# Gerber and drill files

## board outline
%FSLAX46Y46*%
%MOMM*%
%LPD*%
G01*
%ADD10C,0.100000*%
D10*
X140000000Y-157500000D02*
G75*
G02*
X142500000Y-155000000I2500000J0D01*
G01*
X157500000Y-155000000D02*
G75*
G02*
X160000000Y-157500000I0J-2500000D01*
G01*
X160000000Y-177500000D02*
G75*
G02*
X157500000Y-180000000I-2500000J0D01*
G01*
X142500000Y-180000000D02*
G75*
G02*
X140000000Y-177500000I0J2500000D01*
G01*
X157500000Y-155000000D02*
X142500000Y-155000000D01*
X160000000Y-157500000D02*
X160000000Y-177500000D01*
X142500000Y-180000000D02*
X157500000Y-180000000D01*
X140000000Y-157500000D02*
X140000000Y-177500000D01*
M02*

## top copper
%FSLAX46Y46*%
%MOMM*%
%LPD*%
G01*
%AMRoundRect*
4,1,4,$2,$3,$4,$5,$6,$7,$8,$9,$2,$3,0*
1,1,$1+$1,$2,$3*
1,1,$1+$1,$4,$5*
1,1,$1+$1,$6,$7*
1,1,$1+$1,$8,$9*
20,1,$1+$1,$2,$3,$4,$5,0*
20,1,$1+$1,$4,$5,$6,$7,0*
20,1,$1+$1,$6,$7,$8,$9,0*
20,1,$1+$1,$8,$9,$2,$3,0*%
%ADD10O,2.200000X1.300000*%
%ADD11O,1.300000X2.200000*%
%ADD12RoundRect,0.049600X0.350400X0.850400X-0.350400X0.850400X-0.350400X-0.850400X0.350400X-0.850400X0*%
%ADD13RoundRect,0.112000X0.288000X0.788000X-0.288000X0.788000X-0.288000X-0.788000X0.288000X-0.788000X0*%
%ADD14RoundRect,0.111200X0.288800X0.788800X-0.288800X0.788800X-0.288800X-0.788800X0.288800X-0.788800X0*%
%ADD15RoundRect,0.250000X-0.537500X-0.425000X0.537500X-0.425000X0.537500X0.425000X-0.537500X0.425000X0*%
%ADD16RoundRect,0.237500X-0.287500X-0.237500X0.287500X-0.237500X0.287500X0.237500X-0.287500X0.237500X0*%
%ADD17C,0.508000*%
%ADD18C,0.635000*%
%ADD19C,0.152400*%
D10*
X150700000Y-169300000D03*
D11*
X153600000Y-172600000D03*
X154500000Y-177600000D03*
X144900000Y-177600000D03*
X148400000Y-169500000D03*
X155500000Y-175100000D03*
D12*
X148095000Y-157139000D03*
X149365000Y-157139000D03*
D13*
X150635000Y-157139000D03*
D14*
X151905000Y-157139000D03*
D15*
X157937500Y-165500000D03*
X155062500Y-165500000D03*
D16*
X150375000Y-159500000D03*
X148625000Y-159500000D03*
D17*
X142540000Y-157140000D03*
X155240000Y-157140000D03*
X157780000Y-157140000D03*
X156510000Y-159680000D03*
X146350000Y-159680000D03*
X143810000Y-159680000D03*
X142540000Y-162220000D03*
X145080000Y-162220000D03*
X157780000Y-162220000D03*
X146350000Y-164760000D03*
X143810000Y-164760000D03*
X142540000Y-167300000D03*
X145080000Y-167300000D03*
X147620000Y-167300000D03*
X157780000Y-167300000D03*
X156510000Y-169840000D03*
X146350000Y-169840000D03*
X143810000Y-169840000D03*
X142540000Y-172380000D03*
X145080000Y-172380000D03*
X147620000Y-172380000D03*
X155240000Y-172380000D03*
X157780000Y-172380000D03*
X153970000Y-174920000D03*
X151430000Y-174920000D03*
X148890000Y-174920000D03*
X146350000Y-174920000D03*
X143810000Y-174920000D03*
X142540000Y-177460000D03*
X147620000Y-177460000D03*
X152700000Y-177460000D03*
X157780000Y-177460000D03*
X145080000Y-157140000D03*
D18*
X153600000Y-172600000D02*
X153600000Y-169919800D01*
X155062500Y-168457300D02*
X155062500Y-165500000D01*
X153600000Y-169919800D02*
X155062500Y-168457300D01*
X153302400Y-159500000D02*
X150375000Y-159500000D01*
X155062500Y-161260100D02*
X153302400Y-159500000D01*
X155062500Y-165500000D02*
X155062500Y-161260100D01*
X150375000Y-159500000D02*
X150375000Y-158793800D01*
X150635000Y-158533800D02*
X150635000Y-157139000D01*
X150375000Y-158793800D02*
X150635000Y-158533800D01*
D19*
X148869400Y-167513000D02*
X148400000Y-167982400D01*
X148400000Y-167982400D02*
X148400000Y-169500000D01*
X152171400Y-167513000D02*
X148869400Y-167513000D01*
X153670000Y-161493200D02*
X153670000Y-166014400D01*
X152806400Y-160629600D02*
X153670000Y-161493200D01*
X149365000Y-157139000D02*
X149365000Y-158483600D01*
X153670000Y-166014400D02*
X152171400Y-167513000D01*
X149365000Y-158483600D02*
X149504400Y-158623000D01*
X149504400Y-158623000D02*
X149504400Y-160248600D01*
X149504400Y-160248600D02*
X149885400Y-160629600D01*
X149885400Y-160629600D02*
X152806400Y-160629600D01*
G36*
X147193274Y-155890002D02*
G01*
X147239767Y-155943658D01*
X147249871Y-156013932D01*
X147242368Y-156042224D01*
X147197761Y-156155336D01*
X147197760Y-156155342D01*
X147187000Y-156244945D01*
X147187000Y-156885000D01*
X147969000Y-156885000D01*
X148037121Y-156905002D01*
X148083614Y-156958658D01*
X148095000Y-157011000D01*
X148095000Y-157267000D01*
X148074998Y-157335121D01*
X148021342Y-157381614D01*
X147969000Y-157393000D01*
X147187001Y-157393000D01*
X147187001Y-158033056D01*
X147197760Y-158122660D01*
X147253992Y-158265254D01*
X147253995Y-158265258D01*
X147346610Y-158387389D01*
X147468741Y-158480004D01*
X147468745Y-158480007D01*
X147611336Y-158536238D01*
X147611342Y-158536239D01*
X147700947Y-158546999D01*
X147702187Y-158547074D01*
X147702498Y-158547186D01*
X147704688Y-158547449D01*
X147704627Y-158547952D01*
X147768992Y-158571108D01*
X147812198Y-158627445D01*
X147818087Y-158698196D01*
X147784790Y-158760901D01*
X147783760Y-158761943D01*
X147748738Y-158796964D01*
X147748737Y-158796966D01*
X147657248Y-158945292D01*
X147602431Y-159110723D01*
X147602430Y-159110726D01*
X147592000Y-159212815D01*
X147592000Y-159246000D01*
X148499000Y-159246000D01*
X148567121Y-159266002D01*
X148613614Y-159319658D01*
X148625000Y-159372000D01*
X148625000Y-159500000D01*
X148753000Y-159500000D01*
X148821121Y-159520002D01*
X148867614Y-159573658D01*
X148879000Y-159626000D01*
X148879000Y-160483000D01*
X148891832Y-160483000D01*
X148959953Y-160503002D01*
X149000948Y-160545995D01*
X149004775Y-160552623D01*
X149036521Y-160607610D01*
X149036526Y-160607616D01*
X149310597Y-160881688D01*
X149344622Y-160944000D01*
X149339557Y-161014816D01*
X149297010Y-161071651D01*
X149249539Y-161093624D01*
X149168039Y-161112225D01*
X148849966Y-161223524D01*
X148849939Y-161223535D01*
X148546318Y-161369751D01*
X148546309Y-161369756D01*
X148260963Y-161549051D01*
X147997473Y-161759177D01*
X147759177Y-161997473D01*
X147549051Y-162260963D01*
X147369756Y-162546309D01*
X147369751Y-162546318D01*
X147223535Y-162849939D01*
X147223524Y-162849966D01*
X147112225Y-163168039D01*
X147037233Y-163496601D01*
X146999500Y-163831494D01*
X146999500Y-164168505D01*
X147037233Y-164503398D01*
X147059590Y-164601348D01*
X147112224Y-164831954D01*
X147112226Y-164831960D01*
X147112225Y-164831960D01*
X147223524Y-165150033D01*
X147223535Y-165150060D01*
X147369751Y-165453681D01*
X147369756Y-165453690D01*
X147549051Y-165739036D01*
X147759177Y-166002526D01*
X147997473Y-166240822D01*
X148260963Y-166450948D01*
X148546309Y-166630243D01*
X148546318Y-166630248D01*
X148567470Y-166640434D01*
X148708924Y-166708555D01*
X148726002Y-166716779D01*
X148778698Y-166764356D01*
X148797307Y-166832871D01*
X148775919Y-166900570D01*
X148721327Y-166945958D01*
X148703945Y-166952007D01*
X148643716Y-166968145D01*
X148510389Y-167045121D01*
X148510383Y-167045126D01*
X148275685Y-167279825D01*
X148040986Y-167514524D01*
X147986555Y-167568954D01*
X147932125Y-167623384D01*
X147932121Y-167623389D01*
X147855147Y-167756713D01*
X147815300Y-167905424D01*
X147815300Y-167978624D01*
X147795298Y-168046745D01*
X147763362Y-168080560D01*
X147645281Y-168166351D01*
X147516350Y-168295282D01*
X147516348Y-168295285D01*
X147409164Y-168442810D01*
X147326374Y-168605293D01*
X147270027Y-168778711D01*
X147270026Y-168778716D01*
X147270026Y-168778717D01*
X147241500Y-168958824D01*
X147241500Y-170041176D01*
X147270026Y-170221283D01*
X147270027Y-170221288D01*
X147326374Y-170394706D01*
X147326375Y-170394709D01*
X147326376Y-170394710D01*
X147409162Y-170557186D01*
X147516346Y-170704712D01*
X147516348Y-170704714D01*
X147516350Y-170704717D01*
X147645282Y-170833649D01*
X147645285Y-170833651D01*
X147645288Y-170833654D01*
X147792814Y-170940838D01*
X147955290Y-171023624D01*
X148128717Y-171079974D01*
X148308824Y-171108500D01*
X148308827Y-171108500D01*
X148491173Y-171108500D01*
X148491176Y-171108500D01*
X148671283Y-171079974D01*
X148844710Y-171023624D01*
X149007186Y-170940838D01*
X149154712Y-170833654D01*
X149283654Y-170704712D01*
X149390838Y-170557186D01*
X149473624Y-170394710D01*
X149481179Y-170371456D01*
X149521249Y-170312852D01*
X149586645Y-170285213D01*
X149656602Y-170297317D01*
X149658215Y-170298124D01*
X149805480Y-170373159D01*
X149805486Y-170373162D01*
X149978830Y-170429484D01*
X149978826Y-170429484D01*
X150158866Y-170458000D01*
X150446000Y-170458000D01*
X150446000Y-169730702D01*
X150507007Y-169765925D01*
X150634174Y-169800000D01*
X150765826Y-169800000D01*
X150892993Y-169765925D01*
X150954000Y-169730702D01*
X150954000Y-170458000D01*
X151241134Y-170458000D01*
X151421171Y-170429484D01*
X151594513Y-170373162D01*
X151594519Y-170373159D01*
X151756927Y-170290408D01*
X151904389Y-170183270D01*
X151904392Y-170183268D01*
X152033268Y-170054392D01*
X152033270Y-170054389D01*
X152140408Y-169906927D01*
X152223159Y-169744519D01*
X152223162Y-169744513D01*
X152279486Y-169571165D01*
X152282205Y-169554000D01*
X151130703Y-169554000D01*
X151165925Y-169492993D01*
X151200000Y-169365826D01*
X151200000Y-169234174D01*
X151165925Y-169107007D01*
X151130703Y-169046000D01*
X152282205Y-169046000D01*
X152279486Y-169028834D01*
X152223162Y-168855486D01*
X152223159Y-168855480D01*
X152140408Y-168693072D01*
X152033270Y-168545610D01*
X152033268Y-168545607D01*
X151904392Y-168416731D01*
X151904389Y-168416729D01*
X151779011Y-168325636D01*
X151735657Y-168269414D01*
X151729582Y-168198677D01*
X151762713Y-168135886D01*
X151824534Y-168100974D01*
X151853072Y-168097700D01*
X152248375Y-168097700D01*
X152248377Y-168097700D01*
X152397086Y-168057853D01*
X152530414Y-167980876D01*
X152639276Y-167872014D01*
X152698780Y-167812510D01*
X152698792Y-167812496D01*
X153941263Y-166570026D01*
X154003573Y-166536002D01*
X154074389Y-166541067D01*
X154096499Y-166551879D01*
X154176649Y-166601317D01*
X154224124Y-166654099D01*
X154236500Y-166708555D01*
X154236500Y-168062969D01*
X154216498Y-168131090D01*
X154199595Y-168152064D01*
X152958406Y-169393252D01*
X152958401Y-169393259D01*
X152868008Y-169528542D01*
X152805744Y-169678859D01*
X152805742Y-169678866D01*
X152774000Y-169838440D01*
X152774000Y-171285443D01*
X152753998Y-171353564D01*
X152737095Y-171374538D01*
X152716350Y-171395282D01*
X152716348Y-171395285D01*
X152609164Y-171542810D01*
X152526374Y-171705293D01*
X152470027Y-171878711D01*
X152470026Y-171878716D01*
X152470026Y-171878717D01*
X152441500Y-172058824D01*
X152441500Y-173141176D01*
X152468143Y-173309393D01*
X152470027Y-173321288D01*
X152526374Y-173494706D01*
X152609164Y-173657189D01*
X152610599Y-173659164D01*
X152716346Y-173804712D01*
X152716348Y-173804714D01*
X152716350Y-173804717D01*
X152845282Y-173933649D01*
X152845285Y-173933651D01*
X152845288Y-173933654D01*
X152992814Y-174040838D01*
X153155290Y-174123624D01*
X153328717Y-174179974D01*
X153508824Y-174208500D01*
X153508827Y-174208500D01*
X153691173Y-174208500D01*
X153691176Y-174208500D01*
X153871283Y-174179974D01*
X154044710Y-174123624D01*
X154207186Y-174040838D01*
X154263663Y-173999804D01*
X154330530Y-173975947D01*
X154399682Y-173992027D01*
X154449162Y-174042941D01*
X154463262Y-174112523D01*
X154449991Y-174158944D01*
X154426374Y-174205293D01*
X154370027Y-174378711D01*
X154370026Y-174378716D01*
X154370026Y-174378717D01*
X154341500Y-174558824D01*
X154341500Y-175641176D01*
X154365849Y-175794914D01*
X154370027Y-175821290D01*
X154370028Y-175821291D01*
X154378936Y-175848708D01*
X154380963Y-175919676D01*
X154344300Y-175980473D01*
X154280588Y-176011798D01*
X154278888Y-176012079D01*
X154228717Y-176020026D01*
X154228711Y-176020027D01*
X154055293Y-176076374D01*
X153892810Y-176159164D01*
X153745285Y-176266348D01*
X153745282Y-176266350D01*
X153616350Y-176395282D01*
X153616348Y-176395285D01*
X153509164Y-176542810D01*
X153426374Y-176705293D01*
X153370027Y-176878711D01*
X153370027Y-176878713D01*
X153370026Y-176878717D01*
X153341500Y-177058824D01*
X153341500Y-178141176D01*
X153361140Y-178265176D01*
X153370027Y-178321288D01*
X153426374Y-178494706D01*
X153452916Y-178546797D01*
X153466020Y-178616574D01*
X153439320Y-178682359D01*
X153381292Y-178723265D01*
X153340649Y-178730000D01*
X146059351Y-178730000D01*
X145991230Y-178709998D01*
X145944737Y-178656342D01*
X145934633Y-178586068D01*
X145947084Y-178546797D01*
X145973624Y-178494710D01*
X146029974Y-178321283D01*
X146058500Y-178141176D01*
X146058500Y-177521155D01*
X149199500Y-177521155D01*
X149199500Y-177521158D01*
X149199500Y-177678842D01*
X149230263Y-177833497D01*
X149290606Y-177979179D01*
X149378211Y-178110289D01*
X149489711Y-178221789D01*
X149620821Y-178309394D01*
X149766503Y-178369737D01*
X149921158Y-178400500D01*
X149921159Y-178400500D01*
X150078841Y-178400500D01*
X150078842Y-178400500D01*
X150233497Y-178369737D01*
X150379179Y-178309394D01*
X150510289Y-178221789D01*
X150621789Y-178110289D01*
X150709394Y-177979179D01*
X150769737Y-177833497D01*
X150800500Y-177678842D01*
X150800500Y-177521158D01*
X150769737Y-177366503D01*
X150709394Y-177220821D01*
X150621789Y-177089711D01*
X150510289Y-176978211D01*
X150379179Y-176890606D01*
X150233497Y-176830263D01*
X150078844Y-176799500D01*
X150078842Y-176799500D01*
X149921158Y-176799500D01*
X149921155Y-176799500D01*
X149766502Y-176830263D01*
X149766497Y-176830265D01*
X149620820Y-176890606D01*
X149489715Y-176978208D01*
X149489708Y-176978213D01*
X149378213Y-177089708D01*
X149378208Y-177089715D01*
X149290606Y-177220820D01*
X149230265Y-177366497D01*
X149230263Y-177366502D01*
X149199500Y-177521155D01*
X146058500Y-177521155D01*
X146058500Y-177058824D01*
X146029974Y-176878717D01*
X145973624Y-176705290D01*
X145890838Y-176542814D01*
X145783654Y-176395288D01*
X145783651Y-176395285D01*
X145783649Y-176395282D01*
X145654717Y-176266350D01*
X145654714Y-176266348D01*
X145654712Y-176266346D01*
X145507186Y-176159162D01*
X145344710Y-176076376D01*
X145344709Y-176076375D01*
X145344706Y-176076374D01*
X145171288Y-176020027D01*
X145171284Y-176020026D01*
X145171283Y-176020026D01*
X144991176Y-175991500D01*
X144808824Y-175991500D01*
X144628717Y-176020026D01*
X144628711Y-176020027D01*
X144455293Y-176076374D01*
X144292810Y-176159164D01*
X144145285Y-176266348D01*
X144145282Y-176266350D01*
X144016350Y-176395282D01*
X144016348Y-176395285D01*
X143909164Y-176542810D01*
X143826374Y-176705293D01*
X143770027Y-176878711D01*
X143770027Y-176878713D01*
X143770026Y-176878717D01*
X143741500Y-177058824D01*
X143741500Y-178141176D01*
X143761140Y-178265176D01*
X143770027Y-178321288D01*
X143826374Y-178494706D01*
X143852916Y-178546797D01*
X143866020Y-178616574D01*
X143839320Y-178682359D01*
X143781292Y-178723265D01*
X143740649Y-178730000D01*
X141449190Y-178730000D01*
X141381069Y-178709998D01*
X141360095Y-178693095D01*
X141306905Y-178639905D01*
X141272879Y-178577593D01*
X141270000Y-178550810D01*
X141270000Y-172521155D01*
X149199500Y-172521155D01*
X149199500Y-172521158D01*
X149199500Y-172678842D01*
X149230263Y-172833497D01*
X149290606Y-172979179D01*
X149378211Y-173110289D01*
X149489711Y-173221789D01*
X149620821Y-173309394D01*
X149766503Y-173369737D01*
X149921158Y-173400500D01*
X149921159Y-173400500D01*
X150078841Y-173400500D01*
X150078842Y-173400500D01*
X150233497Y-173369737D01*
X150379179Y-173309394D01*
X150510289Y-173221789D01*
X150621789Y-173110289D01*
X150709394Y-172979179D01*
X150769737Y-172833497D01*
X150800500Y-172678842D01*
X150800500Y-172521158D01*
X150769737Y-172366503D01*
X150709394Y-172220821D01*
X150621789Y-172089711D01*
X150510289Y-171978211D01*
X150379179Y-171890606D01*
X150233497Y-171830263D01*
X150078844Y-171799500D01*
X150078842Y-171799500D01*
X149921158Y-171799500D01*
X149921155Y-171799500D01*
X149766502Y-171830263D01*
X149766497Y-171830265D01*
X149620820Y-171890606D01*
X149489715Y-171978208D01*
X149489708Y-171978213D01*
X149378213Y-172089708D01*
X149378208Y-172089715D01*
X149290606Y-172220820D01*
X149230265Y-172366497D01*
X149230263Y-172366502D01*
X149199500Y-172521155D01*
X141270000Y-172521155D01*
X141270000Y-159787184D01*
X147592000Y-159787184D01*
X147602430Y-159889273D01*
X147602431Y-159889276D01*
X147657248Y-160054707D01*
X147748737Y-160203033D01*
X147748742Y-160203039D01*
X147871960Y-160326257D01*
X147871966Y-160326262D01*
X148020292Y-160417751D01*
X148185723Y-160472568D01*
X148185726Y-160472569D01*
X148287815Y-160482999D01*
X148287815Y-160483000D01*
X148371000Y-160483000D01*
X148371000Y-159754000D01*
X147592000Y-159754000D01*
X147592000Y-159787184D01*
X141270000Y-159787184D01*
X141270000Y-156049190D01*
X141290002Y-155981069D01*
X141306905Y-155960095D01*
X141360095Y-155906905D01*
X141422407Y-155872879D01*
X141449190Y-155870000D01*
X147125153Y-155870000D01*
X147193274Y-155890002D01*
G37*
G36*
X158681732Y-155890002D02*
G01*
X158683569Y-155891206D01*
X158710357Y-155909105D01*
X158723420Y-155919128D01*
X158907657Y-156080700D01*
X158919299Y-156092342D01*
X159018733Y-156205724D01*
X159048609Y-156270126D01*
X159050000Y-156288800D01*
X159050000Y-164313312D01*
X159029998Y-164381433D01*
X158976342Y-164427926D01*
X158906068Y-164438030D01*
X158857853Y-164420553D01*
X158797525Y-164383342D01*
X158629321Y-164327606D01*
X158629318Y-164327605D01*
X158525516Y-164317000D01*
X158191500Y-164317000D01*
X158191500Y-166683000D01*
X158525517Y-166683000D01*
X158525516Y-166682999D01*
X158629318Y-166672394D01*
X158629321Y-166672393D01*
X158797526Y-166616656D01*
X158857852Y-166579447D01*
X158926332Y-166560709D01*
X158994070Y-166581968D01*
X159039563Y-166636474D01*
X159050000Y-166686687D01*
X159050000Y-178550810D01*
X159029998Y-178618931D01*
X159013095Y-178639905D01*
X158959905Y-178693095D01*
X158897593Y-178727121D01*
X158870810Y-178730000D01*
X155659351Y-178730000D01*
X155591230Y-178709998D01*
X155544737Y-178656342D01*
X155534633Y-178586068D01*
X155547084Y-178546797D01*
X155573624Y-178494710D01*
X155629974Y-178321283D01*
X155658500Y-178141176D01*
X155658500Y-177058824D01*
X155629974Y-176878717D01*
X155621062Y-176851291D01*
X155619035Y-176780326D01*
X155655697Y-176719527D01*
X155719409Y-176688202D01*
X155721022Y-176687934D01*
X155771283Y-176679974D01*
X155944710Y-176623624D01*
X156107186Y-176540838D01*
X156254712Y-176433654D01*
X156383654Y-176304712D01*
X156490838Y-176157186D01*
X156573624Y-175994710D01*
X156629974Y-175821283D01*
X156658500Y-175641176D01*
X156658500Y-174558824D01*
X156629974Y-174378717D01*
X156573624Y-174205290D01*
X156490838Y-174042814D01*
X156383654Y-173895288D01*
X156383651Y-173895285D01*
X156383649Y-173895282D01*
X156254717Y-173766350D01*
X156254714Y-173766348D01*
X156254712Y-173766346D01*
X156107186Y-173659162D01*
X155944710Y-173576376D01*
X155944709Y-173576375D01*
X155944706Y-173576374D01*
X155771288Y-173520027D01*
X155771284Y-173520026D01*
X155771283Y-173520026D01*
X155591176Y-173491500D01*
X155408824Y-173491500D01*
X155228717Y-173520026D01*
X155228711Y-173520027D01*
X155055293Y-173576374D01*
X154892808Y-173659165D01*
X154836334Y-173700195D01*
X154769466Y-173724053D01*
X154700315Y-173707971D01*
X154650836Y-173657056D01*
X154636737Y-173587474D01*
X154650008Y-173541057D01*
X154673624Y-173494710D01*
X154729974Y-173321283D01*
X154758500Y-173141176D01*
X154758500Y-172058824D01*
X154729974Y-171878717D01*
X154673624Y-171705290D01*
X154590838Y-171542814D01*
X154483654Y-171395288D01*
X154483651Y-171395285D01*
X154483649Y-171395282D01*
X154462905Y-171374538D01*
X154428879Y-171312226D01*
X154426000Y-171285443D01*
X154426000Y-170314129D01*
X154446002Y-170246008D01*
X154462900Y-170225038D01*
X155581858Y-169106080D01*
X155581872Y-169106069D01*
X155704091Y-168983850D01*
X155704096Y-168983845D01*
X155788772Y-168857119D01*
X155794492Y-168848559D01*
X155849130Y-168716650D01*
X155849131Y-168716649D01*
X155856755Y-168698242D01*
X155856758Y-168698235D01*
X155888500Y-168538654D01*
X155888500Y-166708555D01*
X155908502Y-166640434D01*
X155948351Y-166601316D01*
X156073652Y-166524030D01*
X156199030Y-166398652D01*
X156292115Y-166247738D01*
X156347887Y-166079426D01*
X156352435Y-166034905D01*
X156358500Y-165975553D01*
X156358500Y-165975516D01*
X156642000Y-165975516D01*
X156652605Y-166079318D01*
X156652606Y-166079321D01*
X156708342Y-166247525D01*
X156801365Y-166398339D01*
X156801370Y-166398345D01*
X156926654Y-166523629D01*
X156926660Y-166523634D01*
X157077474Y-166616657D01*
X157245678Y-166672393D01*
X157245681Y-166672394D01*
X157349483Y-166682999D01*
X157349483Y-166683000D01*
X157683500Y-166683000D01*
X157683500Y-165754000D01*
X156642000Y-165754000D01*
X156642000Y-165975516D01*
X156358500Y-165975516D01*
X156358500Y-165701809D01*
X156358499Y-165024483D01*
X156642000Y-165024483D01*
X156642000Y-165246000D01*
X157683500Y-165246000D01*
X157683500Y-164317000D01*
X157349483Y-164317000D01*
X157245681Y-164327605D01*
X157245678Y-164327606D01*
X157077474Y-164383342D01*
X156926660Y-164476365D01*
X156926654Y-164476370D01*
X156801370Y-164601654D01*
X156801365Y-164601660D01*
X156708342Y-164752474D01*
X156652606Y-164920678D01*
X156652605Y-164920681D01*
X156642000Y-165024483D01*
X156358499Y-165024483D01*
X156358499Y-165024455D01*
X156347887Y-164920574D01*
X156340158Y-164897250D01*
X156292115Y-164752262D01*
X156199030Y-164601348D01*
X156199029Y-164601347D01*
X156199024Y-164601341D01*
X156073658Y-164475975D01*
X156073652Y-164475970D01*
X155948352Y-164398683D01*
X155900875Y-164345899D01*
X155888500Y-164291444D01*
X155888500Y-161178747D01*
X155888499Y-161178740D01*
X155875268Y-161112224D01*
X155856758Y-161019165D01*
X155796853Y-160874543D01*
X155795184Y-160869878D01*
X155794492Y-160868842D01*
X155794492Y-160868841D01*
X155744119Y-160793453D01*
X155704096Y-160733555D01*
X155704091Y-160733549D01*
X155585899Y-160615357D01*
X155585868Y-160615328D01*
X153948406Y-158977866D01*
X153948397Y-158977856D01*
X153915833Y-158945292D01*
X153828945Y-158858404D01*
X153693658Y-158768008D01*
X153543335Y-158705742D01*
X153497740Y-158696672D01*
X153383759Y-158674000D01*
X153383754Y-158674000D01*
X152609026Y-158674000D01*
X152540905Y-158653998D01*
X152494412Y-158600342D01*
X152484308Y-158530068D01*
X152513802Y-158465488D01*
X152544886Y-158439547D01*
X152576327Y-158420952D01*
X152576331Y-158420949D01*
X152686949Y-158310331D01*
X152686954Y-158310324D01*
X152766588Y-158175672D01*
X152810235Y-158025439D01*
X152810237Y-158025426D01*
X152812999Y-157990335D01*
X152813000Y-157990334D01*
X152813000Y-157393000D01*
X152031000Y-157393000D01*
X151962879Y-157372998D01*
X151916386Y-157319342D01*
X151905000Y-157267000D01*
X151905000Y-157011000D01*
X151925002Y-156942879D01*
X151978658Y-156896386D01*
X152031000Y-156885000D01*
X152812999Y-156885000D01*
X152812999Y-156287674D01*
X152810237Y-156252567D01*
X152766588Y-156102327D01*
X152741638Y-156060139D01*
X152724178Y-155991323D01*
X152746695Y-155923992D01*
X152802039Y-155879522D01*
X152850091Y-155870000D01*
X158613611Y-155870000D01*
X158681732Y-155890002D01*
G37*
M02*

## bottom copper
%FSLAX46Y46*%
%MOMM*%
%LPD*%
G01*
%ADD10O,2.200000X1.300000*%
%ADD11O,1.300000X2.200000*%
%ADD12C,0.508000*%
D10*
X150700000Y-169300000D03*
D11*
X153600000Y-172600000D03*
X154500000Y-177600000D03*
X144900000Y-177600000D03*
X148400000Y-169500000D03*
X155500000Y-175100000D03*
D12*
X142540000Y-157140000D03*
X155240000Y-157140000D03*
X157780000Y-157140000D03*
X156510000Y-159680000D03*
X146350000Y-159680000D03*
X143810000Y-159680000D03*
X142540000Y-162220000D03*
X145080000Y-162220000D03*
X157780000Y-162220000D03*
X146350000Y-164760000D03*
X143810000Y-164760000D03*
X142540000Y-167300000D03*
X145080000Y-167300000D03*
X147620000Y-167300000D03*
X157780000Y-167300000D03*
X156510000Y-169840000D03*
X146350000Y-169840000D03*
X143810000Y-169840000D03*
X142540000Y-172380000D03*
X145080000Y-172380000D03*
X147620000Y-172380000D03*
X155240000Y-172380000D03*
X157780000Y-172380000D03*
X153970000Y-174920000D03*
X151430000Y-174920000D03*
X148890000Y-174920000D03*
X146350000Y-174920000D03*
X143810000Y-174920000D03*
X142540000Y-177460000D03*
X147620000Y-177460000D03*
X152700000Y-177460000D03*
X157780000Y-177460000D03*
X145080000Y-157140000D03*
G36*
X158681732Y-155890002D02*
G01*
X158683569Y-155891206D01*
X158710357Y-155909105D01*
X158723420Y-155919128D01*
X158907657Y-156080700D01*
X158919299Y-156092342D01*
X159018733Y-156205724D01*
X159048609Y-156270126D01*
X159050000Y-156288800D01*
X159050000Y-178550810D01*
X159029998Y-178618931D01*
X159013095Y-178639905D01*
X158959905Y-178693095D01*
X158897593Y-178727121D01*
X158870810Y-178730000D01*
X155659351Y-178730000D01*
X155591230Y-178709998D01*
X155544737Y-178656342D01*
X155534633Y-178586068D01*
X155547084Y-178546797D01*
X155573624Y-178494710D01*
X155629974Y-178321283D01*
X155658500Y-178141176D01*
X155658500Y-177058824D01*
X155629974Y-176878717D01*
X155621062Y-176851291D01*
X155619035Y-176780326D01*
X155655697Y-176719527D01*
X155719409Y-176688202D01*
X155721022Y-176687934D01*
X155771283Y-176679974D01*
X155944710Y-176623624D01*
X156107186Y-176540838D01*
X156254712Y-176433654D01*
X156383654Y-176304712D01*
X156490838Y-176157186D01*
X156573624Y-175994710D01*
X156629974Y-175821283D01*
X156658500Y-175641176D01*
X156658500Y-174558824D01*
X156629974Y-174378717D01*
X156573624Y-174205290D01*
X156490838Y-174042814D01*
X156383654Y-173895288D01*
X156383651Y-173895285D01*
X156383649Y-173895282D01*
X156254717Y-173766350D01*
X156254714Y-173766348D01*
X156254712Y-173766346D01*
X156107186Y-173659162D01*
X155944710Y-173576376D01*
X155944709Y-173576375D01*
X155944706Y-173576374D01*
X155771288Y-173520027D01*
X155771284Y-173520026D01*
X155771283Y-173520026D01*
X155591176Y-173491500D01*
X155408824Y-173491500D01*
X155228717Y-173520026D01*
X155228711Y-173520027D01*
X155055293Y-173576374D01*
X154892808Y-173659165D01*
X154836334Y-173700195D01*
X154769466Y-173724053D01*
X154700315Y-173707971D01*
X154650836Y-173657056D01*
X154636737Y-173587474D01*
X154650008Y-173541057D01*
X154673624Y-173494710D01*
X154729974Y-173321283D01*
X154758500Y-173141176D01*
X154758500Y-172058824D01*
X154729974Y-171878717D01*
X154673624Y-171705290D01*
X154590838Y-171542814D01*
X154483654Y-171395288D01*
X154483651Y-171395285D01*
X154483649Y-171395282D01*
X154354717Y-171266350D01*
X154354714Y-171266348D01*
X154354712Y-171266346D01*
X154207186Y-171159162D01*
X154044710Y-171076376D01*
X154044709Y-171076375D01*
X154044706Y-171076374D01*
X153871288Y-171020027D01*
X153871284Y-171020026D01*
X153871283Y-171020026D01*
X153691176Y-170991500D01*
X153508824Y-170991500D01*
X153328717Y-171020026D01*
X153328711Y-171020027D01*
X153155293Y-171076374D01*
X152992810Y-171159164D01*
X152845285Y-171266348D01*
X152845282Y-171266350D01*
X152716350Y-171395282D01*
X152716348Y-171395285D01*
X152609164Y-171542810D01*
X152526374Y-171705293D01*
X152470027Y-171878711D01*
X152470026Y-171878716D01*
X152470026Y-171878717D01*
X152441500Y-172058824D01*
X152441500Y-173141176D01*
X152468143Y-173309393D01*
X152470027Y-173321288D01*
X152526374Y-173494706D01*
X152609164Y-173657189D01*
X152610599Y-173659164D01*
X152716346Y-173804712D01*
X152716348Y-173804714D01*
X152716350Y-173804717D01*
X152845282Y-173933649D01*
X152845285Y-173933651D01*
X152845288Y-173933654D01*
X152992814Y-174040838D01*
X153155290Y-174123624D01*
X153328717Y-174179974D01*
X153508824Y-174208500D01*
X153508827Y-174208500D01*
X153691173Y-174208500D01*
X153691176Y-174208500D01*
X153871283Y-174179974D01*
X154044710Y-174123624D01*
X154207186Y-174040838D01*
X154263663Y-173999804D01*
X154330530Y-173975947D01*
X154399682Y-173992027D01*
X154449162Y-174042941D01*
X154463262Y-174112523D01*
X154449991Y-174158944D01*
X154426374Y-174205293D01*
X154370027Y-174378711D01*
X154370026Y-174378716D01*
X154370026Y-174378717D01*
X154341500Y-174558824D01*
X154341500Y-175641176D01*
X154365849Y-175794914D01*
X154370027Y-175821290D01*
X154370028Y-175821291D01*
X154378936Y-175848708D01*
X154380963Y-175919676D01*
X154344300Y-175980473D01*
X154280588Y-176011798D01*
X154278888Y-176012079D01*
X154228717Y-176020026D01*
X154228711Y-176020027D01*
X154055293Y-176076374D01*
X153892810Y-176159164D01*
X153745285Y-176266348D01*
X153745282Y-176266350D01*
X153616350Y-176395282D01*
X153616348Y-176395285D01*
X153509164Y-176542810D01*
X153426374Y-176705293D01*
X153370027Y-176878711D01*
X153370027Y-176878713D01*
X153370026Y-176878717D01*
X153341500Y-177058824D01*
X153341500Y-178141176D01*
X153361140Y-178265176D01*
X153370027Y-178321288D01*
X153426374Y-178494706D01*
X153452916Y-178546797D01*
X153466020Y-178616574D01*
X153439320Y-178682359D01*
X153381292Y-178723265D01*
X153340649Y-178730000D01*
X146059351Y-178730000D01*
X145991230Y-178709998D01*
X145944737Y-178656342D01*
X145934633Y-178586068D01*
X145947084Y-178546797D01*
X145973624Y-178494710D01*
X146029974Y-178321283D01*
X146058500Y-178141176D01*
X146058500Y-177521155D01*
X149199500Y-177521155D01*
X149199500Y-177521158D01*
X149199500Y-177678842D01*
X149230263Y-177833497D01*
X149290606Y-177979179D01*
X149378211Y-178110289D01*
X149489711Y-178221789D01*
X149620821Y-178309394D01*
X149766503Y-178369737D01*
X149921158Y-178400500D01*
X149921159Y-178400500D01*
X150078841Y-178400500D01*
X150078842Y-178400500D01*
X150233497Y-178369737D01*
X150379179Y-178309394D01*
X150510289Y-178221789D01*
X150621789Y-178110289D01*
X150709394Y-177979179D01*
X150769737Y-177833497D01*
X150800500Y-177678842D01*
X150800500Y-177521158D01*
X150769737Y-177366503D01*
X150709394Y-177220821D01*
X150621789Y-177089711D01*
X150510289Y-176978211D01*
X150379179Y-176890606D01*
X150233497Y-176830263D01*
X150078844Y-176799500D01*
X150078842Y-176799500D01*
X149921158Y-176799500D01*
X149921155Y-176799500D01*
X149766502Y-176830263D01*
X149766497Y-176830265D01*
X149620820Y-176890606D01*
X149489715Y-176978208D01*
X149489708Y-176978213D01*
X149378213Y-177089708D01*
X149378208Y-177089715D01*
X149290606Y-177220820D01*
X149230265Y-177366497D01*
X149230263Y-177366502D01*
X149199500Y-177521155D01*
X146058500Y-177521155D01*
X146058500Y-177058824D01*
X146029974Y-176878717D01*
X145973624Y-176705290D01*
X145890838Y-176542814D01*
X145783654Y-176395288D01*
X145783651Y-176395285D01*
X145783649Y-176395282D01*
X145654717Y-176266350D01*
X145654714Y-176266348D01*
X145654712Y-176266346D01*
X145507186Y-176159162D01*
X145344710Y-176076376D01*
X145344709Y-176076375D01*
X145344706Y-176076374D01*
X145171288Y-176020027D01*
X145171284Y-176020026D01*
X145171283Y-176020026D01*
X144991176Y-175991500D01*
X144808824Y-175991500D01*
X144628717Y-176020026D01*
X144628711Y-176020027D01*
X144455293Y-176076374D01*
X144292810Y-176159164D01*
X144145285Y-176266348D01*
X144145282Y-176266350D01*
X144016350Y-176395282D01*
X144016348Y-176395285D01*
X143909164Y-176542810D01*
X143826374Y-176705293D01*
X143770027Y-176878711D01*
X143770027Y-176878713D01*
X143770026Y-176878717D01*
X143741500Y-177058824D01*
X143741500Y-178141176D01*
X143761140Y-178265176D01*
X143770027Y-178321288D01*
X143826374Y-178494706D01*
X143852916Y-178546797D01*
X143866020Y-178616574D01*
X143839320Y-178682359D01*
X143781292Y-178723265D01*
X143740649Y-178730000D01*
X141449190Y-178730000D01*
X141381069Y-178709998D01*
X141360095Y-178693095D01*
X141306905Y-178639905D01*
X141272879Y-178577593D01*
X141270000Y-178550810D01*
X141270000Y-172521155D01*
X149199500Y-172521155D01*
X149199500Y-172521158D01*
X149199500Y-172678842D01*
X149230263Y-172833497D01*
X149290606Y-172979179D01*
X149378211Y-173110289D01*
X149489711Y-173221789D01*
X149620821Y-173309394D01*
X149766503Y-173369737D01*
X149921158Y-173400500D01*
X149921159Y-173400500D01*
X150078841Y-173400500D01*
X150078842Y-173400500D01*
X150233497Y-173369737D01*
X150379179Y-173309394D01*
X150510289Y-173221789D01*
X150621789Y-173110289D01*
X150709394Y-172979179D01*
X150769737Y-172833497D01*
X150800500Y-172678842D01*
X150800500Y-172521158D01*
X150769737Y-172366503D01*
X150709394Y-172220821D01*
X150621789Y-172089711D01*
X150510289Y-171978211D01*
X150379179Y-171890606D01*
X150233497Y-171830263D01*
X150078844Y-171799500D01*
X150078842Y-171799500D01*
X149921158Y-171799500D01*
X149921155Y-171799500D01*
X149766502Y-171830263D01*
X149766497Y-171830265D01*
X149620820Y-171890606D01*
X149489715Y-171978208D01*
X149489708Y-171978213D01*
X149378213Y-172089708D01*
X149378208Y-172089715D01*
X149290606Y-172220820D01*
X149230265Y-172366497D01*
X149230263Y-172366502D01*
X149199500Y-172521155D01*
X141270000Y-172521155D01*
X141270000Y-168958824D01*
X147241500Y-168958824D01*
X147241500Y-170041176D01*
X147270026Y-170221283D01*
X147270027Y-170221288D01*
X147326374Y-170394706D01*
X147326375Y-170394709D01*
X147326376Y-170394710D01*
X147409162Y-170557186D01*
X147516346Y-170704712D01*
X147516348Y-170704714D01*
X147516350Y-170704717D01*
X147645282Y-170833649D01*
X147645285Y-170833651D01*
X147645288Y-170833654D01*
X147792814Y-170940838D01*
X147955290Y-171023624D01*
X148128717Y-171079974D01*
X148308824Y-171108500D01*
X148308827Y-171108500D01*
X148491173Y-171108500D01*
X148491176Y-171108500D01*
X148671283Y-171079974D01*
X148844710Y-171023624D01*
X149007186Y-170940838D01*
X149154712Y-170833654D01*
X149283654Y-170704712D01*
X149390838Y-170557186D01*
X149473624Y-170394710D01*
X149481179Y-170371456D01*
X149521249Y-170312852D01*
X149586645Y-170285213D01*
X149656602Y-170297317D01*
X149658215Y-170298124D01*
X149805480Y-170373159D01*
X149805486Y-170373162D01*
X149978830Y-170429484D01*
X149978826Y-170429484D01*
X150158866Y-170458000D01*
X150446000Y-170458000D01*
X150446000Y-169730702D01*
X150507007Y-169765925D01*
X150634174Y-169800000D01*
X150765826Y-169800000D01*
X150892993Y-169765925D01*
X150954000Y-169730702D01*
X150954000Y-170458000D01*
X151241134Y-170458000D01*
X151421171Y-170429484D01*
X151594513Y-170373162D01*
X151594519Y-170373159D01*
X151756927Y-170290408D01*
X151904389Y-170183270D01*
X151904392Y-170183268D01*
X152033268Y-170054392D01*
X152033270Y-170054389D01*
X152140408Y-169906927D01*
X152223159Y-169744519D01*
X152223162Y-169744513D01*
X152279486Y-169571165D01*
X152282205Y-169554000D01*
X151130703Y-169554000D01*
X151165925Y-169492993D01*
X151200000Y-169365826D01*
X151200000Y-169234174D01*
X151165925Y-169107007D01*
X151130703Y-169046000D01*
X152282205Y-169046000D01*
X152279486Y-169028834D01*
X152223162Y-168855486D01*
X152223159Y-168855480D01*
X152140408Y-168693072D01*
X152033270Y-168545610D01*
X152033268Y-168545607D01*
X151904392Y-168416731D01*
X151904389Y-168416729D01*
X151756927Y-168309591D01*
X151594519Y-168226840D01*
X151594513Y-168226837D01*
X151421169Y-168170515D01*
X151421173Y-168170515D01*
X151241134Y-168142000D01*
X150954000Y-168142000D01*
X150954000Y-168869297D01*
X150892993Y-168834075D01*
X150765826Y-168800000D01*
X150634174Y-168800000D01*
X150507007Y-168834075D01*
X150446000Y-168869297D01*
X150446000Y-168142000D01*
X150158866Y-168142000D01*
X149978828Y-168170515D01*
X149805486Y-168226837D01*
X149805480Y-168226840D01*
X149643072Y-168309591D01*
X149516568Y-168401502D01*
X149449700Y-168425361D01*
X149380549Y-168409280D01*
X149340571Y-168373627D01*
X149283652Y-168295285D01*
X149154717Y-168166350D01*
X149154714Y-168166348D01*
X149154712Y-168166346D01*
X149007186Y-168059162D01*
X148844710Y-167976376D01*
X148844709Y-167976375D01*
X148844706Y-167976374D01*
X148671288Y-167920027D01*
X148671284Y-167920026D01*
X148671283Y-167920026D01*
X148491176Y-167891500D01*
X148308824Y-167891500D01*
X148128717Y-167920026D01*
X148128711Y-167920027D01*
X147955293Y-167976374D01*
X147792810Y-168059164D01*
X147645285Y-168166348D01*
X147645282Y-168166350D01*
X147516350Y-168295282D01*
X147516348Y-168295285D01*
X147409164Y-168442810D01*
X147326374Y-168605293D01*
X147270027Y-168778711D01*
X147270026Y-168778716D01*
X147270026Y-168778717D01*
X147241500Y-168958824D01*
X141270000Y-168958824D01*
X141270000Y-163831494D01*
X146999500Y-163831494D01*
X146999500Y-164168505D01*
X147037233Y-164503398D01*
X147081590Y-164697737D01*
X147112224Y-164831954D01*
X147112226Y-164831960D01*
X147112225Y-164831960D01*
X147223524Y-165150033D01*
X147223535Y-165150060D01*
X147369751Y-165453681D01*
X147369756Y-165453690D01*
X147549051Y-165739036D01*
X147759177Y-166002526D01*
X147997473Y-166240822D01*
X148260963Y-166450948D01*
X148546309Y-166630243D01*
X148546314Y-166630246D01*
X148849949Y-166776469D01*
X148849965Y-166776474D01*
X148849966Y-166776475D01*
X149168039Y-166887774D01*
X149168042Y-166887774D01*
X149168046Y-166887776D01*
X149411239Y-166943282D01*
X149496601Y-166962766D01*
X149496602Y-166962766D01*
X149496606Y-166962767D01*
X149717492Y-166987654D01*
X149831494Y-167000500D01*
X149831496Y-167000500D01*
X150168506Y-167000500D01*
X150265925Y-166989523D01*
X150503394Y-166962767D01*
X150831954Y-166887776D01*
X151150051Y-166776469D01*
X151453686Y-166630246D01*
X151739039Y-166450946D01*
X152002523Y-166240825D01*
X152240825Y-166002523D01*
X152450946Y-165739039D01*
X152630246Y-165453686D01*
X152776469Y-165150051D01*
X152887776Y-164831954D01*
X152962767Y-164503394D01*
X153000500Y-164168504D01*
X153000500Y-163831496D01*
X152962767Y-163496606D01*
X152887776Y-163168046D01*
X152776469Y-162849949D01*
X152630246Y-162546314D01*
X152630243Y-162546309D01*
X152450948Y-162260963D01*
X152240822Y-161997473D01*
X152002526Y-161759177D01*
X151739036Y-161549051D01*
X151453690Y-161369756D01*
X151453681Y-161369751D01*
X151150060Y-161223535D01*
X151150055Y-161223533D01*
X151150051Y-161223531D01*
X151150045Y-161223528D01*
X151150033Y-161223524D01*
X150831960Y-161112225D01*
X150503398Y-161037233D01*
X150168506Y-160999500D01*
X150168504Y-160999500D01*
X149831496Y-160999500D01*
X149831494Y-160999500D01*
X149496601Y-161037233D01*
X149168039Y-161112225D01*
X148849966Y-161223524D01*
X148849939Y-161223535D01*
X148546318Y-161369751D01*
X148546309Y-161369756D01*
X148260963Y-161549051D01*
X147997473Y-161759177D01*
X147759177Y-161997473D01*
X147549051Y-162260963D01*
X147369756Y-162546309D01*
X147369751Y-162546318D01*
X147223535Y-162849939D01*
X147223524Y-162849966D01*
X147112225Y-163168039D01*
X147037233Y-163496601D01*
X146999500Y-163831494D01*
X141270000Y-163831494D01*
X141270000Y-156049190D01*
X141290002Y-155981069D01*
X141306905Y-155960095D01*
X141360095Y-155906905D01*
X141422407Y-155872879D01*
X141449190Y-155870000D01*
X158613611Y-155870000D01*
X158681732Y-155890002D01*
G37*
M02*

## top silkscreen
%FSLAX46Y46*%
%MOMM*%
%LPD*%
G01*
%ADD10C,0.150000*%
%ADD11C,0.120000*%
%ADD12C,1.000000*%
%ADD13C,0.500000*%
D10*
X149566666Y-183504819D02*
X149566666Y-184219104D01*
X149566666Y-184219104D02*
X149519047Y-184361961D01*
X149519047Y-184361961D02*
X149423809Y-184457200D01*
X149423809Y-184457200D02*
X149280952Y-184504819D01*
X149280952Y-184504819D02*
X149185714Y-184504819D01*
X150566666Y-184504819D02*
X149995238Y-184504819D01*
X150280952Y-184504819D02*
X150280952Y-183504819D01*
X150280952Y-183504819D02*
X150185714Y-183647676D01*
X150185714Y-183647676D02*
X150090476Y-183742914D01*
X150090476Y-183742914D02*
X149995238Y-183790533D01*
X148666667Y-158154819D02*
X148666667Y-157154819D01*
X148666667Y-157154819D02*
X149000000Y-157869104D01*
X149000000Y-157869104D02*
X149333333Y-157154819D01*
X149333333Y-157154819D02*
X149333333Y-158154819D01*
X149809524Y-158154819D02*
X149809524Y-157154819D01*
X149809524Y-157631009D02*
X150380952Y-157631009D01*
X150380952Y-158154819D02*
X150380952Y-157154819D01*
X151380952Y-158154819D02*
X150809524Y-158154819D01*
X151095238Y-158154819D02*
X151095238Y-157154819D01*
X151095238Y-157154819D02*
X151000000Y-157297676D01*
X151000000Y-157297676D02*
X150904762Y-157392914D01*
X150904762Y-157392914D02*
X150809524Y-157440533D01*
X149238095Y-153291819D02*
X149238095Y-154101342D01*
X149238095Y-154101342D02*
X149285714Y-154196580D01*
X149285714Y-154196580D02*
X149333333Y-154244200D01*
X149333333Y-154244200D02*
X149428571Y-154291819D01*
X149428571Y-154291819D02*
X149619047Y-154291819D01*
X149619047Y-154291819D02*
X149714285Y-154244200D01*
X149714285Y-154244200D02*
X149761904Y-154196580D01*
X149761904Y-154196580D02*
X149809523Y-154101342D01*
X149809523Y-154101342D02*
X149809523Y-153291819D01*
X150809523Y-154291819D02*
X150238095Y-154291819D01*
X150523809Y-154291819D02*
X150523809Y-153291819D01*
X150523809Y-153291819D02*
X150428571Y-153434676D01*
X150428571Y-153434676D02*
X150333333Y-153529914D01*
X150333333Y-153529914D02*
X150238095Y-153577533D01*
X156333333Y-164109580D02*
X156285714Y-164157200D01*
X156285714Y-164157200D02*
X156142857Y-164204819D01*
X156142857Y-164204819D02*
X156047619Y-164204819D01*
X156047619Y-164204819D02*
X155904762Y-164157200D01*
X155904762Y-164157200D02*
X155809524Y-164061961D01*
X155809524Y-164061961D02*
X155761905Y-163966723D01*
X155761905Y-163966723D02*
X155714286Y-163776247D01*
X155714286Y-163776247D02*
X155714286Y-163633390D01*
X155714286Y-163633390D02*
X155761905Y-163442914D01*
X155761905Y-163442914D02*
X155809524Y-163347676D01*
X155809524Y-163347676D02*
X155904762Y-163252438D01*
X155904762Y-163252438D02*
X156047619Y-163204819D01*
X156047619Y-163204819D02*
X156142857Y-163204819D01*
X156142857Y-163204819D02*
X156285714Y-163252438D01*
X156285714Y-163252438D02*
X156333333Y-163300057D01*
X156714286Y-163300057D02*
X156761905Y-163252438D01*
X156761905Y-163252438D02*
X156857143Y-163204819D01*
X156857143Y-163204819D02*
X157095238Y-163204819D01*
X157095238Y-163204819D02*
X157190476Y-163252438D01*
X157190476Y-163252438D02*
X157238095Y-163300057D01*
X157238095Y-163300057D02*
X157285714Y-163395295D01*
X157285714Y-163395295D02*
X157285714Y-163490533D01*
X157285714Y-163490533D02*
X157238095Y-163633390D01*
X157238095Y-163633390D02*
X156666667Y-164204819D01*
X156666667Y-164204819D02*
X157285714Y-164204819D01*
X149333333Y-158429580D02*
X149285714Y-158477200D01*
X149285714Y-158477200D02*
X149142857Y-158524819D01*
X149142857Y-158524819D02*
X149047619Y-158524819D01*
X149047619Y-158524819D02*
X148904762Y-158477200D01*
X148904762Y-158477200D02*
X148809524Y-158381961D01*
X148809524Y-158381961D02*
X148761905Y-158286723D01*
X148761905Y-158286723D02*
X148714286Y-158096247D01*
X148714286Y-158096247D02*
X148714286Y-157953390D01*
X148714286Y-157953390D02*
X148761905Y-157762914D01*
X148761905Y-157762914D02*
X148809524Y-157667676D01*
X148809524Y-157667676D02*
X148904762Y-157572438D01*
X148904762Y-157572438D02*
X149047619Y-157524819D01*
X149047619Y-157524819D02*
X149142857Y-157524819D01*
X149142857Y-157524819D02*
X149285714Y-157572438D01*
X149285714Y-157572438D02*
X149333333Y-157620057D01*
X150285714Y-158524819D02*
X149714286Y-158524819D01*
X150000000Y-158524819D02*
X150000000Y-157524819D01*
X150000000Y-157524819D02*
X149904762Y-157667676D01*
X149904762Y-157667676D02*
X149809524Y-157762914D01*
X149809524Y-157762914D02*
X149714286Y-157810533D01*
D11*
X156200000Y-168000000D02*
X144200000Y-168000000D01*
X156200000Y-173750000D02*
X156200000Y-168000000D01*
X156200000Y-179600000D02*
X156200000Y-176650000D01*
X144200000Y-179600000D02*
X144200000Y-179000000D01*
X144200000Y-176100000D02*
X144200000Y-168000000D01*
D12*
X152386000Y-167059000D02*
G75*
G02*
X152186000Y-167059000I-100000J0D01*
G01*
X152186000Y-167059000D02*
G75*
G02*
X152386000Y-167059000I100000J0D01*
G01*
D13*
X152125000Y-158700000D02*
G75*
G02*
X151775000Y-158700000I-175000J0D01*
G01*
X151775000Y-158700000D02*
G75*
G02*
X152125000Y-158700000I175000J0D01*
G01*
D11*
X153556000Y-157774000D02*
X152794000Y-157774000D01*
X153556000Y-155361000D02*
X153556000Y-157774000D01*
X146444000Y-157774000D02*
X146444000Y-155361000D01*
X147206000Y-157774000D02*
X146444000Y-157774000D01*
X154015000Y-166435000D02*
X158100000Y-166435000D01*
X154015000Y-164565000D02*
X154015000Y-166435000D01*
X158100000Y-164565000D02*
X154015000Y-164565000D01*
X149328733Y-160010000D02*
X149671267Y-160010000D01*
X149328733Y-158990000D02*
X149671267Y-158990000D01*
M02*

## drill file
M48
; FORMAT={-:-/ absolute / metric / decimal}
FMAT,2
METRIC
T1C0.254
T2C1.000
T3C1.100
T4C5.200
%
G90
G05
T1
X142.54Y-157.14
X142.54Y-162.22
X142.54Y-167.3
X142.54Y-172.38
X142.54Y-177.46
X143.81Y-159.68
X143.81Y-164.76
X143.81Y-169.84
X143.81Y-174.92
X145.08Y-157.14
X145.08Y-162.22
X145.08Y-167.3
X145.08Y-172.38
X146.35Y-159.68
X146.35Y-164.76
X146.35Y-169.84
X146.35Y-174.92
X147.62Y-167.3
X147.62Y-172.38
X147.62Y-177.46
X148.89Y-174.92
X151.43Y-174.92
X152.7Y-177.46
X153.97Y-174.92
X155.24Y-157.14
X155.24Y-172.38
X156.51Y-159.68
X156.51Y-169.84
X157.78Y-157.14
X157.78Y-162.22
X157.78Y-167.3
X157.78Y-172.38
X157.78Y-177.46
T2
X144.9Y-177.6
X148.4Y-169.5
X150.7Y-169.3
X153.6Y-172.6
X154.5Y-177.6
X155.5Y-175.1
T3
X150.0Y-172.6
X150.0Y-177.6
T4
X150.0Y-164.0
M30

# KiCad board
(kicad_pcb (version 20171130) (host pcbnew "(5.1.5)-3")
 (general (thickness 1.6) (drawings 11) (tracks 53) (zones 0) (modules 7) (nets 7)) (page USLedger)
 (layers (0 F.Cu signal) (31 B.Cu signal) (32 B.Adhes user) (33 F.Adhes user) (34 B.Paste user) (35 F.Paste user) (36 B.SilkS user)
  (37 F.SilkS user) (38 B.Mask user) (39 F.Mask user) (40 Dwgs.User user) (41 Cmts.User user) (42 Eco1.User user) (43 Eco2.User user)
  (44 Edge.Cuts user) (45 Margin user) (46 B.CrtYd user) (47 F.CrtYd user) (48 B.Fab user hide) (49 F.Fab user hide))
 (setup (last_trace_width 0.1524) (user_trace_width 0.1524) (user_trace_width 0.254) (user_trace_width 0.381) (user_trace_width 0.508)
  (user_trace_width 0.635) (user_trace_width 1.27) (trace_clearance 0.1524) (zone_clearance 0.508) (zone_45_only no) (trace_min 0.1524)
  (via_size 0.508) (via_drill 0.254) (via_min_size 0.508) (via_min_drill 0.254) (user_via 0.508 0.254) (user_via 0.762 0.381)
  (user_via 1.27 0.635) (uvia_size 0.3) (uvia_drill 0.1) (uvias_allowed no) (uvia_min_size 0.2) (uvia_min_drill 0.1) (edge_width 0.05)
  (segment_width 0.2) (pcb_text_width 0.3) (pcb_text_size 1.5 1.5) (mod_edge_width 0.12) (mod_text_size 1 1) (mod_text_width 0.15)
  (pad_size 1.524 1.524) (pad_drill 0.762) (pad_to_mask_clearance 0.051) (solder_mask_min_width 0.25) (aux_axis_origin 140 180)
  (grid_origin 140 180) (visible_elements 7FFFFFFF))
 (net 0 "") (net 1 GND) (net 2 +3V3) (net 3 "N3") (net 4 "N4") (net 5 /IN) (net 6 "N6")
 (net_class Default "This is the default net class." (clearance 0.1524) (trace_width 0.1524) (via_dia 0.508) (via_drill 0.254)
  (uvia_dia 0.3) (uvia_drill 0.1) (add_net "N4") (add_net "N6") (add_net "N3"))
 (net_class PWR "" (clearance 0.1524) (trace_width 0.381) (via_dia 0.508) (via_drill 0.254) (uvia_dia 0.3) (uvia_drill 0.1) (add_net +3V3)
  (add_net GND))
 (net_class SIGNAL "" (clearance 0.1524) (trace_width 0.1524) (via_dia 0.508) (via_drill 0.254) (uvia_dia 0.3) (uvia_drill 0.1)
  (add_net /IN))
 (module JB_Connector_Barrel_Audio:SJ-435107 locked (layer F.Cu) (at 150 177.6 180)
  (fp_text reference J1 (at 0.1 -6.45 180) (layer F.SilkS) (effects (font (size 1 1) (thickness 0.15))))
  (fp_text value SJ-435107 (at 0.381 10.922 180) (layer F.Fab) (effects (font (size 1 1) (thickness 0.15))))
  (fp_line (start -6.2 9.6) (end 5.8 9.6) (layer F.SilkS) (width 0.12))
  (fp_line (start -6.2 3.85) (end -6.2 9.6) (layer F.SilkS) (width 0.12))
  (fp_line (start -6.2 -2) (end -6.2 0.95) (layer F.SilkS) (width 0.12))
  (fp_line (start 5.8 -2) (end 5.8 -1.4) (layer F.SilkS) (width 0.12))
  (fp_line (start 5.8 1.5) (end 5.8 9.6) (layer F.SilkS) (width 0.12))
  (fp_circle (center -2.286 10.541) (end -2.186 10.541) (layer F.SilkS) (width 1))
  (pad S thru_hole oval (at -0.7 8.3 180) (size 2.2 1.3) (drill 1) (layers *.Cu *.Mask) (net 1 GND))
  (pad T thru_hole oval (at -3.6 5 270) (size 2.2 1.3) (drill 1) (layers *.Cu *.Mask) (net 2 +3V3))
  (pad R2 thru_hole oval (at -4.5 0 270) (size 2.2 1.3) (drill 1) (layers *.Cu *.Mask) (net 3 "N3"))
  (pad G1 thru_hole oval (at 5.1 0 270) (size 2.2 1.3) (drill 1) (layers *.Cu *.Mask) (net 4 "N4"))
  (pad R1 thru_hole oval (at 1.6 8.1 270) (size 2.2 1.3) (drill 1) (layers *.Cu *.Mask) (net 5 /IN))
  (pad "" np_thru_hole circle (at 0 0 180) (size 1.1 1.1) (drill 1.1) (layers *.Cu *.Mask))
  (pad "" np_thru_hole circle (at 0 5 180) (size 1.1 1.1) (drill 1.1) (layers *.Cu *.Mask))
  (pad G2 thru_hole oval (at -5.5 2.5 270) (size 2.2 1.3) (drill 1) (layers *.Cu *.Mask) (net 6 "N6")))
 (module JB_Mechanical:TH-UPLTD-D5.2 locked (layer F.Cu) (at 150 164)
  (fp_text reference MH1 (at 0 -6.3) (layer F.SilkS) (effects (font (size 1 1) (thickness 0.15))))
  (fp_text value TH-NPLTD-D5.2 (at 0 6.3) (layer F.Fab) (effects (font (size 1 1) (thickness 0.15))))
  (pad "" np_thru_hole circle (at 0 0) (size 5.2 5.2) (drill 5.2) (layers *.Cu *.Mask) (clearance 0.4)))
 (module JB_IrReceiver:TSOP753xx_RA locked (layer F.Cu) (at 150 156.25 180)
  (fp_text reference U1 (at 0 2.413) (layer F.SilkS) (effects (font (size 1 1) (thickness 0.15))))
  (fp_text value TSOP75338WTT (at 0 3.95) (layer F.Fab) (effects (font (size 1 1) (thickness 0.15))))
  (fp_circle (center -1.95 -2.45) (end -1.775 -2.45) (layer F.SilkS) (width 0.5))
  (fp_line (start -3.556 -1.524) (end -2.794 -1.524) (layer F.SilkS) (width 0.12))
  (fp_line (start -3.556 0.889) (end -3.556 -1.524) (layer F.SilkS) (width 0.12))
  (fp_line (start 3.556 -1.524) (end 3.556 0.889) (layer F.SilkS) (width 0.12))
  (fp_line (start 2.794 -1.524) (end 3.556 -1.524) (layer F.SilkS) (width 0.12))
  (pad 4 smd roundrect (at 1.905 -0.889 180) (size 0.8 1.8) (layers F.Cu F.Paste F.Mask) (roundrect_rratio 0.062) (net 1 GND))
  (pad 3 smd roundrect (at 0.635 -0.889 180) (size 0.8 1.8) (layers F.Cu F.Paste F.Mask) (roundrect_rratio 0.062) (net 5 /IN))
  (pad 2 smd roundrect (at -0.635 -0.889 180) (size 0.8 1.8) (layers F.Cu F.Paste F.Mask) (roundrect_rratio 0.14) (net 2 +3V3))
  (pad 1 smd roundrect (at -1.905 -0.889 180) (size 0.8 1.8) (layers F.Cu F.Paste F.Mask) (roundrect_rratio 0.139) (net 1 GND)))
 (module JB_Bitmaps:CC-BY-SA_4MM (layer B.Cu) (at 143.81 169.205 180)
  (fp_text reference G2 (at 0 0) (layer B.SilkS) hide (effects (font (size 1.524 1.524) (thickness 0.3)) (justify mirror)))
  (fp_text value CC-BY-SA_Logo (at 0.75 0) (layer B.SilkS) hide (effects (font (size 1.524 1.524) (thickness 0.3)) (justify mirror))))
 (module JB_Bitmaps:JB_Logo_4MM (layer B.Cu) (at 143.937 165.268 180)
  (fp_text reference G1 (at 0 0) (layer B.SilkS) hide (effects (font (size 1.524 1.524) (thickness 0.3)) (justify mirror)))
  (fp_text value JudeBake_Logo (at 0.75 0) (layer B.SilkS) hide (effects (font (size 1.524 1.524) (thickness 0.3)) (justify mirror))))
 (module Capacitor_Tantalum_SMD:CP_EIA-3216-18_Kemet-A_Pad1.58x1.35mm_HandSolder (layer F.Cu) (at 156.5 165.5)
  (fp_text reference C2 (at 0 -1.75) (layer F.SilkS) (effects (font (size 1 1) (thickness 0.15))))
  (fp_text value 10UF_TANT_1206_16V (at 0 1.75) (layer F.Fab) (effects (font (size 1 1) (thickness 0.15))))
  (fp_line (start -2.485 0.935) (end 1.6 0.935) (layer F.SilkS) (width 0.12))
  (fp_line (start -2.485 -0.935) (end -2.485 0.935) (layer F.SilkS) (width 0.12))
  (fp_line (start 1.6 -0.935) (end -2.485 -0.935) (layer F.SilkS) (width 0.12))
  (pad 2 smd roundrect (at 1.4375 0) (size 1.575 1.35) (layers F.Cu F.Paste F.Mask) (roundrect_rratio 0.185185) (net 1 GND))
  (pad 1 smd roundrect (at -1.4375 0) (size 1.575 1.35) (layers F.Cu F.Paste F.Mask) (roundrect_rratio 0.185185) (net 2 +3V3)))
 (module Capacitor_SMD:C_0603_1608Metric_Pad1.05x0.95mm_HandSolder (layer F.Cu) (at 149.5 159.5)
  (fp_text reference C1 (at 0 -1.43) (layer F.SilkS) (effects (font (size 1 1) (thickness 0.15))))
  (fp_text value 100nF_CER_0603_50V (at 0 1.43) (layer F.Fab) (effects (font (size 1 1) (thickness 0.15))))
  (fp_line (start -0.171267 0.51) (end 0.171267 0.51) (layer F.SilkS) (width 0.12))
  (fp_line (start -0.171267 -0.51) (end 0.171267 -0.51) (layer F.SilkS) (width 0.12))
  (pad 2 smd roundrect (at 0.875 0) (size 1.05 0.95) (layers F.Cu F.Paste F.Mask) (roundrect_rratio 0.25) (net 2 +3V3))
  (pad 1 smd roundrect (at -0.875 0) (size 1.05 0.95) (layers F.Cu F.Paste F.Mask) (roundrect_rratio 0.25) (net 1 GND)))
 (gr_arc (start 142.5 157.5) (end 142.5 155) (angle -90) (layer Edge.Cuts) (width 0.1))
 (gr_arc (start 157.5 157.5) (end 160 157.5) (angle -90) (layer Edge.Cuts) (width 0.1))
 (gr_arc (start 157.5 177.5) (end 157.5 180) (angle -90) (layer Edge.Cuts) (width 0.1))
 (gr_arc (start 142.5 177.5) (end 140 177.5) (angle -90) (layer Edge.Cuts) (width 0.1))
 (gr_line (start 157.5 155) (end 142.5 155) (layer Edge.Cuts) (width 0.1))
 (gr_line (start 160 157.5) (end 160 177.5) (layer Edge.Cuts) (width 0.1))
 (gr_line (start 142.5 180) (end 157.5 180) (layer Edge.Cuts) (width 0.1))
 (gr_line (start 140 157.5) (end 140 177.5) (layer Edge.Cuts) (width 0.1))
 (segment (start 153.6 172.6) (end 153.6 169.9198) (width 0.635) (layer F.Cu) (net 2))
 (segment (start 155.0625 168.4573) (end 155.0625 165.5) (width 0.635) (layer F.Cu) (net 2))
 (segment (start 153.6 169.9198) (end 155.0625 168.4573) (width 0.635) (layer F.Cu) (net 2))
 (segment (start 153.3024 159.5) (end 150.375 159.5) (width 0.635) (layer F.Cu) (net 2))
 (segment (start 155.0625 161.2601) (end 153.3024 159.5) (width 0.635) (layer F.Cu) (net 2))
 (segment (start 155.0625 165.5) (end 155.0625 161.2601) (width 0.635) (layer F.Cu) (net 2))
 (segment (start 150.375 159.5) (end 150.375 158.7938) (width 0.635) (layer F.Cu) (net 2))
 (segment (start 150.635 158.5338) (end 150.635 157.139) (width 0.635) (layer F.Cu) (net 2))
 (segment (start 150.375 158.7938) (end 150.635 158.5338) (width 0.635) (layer F.Cu) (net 2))
 (via (at 142.54 157.14) (size 0.508) (drill 0.254) (layers F.Cu B.Cu) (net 1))
 (via (at 155.24 157.14) (size 0.508) (drill 0.254) (layers F.Cu B.Cu) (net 1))
 (via (at 157.78 157.14) (size 0.508) (drill 0.254) (layers F.Cu B.Cu) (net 1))
 (via (at 156.51 159.68) (size 0.508) (drill 0.254) (layers F.Cu B.Cu) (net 1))
 (via (at 146.35 159.68) (size 0.508) (drill 0.254) (layers F.Cu B.Cu) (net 1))
 (via (at 143.81 159.68) (size 0.508) (drill 0.254) (layers F.Cu B.Cu) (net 1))
 (via (at 142.54 162.22) (size 0.508) (drill 0.254) (layers F.Cu B.Cu) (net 1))
 (via (at 145.08 162.22) (size 0.508) (drill 0.254) (layers F.Cu B.Cu) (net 1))
 (via (at 157.78 162.22) (size 0.508) (drill 0.254) (layers F.Cu B.Cu) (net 1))
 (via (at 146.35 164.76) (size 0.508) (drill 0.254) (layers F.Cu B.Cu) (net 1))
 (via (at 143.81 164.76) (size 0.508) (drill 0.254) (layers F.Cu B.Cu) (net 1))
 (via (at 142.54 167.3) (size 0.508) (drill 0.254) (layers F.Cu B.Cu) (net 1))
 (via (at 145.08 167.3) (size 0.508) (drill 0.254) (layers F.Cu B.Cu) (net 1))
 (via (at 147.62 167.3) (size 0.508) (drill 0.254) (layers F.Cu B.Cu) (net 1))
 (via (at 157.78 167.3) (size 0.508) (drill 0.254) (layers F.Cu B.Cu) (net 1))
 (via (at 156.51 169.84) (size 0.508) (drill 0.254) (layers F.Cu B.Cu) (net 1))
 (via (at 146.35 169.84) (size 0.508) (drill 0.254) (layers F.Cu B.Cu) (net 1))
 (via (at 143.81 169.84) (size 0.508) (drill 0.254) (layers F.Cu B.Cu) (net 1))
 (via (at 142.54 172.38) (size 0.508) (drill 0.254) (layers F.Cu B.Cu) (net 1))
 (via (at 145.08 172.38) (size 0.508) (drill 0.254) (layers F.Cu B.Cu) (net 1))
 (via (at 147.62 172.38) (size 0.508) (drill 0.254) (layers F.Cu B.Cu) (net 1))
 (via (at 155.24 172.38) (size 0.508) (drill 0.254) (layers F.Cu B.Cu) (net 1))
 (via (at 157.78 172.38) (size 0.508) (drill 0.254) (layers F.Cu B.Cu) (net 1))
 (via (at 153.97 174.92) (size 0.508) (drill 0.254) (layers F.Cu B.Cu) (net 1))
 (via (at 151.43 174.92) (size 0.508) (drill 0.254) (layers F.Cu B.Cu) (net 1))
 (via (at 148.89 174.92) (size 0.508) (drill 0.254) (layers F.Cu B.Cu) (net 1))
 (via (at 146.35 174.92) (size 0.508) (drill 0.254) (layers F.Cu B.Cu) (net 1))
 (via (at 143.81 174.92) (size 0.508) (drill 0.254) (layers F.Cu B.Cu) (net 1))
 (via (at 142.54 177.46) (size 0.508) (drill 0.254) (layers F.Cu B.Cu) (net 1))
 (via (at 147.62 177.46) (size 0.508) (drill 0.254) (layers F.Cu B.Cu) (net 1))
 (via (at 152.7 177.46) (size 0.508) (drill 0.254) (layers F.Cu B.Cu) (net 1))
 (via (at 157.78 177.46) (size 0.508) (drill 0.254) (layers F.Cu B.Cu) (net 1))
 (via (at 145.08 157.14) (size 0.508) (drill 0.254) (layers F.Cu B.Cu) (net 1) (status 1000000))
 (segment (start 148.8694 167.513) (end 148.4 167.9824) (width 0.1524) (layer F.Cu) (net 5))
 (segment (start 148.4 167.9824) (end 148.4 169.5) (width 0.1524) (layer F.Cu) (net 5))
 (segment (start 152.1714 167.513) (end 148.8694 167.513) (width 0.1524) (layer F.Cu) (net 5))
 (segment (start 153.67 161.4932) (end 153.67 166.0144) (width 0.1524) (layer F.Cu) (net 5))
 (segment (start 152.8064 160.6296) (end 153.67 161.4932) (width 0.1524) (layer F.Cu) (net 5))
 (segment (start 149.365 157.139) (end 149.365 158.4836) (width 0.1524) (layer F.Cu) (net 5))
 (segment (start 153.67 166.0144) (end 152.1714 167.513) (width 0.1524) (layer F.Cu) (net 5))
 (segment (start 149.365 158.4836) (end 149.5044 158.623) (width 0.1524) (layer F.Cu) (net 5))
 (segment (start 149.5044 158.623) (end 149.5044 160.2486) (width 0.1524) (layer F.Cu) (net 5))
 (segment (start 149.5044 160.2486) (end 149.8854 160.6296) (width 0.1524) (layer F.Cu) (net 5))
 (segment (start 149.8854 160.6296) (end 152.8064 160.6296) (width 0.1524) (layer F.Cu) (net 5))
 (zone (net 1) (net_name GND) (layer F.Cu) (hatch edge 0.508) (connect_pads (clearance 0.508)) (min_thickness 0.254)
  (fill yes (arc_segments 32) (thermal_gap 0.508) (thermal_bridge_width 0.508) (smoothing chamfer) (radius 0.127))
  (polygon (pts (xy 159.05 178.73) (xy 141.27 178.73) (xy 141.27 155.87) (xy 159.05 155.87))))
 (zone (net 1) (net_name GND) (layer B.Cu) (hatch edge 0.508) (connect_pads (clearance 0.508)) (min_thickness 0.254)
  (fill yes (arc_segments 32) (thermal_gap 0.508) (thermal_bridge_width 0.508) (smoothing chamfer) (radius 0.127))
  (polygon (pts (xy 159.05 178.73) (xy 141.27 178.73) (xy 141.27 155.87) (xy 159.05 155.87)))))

